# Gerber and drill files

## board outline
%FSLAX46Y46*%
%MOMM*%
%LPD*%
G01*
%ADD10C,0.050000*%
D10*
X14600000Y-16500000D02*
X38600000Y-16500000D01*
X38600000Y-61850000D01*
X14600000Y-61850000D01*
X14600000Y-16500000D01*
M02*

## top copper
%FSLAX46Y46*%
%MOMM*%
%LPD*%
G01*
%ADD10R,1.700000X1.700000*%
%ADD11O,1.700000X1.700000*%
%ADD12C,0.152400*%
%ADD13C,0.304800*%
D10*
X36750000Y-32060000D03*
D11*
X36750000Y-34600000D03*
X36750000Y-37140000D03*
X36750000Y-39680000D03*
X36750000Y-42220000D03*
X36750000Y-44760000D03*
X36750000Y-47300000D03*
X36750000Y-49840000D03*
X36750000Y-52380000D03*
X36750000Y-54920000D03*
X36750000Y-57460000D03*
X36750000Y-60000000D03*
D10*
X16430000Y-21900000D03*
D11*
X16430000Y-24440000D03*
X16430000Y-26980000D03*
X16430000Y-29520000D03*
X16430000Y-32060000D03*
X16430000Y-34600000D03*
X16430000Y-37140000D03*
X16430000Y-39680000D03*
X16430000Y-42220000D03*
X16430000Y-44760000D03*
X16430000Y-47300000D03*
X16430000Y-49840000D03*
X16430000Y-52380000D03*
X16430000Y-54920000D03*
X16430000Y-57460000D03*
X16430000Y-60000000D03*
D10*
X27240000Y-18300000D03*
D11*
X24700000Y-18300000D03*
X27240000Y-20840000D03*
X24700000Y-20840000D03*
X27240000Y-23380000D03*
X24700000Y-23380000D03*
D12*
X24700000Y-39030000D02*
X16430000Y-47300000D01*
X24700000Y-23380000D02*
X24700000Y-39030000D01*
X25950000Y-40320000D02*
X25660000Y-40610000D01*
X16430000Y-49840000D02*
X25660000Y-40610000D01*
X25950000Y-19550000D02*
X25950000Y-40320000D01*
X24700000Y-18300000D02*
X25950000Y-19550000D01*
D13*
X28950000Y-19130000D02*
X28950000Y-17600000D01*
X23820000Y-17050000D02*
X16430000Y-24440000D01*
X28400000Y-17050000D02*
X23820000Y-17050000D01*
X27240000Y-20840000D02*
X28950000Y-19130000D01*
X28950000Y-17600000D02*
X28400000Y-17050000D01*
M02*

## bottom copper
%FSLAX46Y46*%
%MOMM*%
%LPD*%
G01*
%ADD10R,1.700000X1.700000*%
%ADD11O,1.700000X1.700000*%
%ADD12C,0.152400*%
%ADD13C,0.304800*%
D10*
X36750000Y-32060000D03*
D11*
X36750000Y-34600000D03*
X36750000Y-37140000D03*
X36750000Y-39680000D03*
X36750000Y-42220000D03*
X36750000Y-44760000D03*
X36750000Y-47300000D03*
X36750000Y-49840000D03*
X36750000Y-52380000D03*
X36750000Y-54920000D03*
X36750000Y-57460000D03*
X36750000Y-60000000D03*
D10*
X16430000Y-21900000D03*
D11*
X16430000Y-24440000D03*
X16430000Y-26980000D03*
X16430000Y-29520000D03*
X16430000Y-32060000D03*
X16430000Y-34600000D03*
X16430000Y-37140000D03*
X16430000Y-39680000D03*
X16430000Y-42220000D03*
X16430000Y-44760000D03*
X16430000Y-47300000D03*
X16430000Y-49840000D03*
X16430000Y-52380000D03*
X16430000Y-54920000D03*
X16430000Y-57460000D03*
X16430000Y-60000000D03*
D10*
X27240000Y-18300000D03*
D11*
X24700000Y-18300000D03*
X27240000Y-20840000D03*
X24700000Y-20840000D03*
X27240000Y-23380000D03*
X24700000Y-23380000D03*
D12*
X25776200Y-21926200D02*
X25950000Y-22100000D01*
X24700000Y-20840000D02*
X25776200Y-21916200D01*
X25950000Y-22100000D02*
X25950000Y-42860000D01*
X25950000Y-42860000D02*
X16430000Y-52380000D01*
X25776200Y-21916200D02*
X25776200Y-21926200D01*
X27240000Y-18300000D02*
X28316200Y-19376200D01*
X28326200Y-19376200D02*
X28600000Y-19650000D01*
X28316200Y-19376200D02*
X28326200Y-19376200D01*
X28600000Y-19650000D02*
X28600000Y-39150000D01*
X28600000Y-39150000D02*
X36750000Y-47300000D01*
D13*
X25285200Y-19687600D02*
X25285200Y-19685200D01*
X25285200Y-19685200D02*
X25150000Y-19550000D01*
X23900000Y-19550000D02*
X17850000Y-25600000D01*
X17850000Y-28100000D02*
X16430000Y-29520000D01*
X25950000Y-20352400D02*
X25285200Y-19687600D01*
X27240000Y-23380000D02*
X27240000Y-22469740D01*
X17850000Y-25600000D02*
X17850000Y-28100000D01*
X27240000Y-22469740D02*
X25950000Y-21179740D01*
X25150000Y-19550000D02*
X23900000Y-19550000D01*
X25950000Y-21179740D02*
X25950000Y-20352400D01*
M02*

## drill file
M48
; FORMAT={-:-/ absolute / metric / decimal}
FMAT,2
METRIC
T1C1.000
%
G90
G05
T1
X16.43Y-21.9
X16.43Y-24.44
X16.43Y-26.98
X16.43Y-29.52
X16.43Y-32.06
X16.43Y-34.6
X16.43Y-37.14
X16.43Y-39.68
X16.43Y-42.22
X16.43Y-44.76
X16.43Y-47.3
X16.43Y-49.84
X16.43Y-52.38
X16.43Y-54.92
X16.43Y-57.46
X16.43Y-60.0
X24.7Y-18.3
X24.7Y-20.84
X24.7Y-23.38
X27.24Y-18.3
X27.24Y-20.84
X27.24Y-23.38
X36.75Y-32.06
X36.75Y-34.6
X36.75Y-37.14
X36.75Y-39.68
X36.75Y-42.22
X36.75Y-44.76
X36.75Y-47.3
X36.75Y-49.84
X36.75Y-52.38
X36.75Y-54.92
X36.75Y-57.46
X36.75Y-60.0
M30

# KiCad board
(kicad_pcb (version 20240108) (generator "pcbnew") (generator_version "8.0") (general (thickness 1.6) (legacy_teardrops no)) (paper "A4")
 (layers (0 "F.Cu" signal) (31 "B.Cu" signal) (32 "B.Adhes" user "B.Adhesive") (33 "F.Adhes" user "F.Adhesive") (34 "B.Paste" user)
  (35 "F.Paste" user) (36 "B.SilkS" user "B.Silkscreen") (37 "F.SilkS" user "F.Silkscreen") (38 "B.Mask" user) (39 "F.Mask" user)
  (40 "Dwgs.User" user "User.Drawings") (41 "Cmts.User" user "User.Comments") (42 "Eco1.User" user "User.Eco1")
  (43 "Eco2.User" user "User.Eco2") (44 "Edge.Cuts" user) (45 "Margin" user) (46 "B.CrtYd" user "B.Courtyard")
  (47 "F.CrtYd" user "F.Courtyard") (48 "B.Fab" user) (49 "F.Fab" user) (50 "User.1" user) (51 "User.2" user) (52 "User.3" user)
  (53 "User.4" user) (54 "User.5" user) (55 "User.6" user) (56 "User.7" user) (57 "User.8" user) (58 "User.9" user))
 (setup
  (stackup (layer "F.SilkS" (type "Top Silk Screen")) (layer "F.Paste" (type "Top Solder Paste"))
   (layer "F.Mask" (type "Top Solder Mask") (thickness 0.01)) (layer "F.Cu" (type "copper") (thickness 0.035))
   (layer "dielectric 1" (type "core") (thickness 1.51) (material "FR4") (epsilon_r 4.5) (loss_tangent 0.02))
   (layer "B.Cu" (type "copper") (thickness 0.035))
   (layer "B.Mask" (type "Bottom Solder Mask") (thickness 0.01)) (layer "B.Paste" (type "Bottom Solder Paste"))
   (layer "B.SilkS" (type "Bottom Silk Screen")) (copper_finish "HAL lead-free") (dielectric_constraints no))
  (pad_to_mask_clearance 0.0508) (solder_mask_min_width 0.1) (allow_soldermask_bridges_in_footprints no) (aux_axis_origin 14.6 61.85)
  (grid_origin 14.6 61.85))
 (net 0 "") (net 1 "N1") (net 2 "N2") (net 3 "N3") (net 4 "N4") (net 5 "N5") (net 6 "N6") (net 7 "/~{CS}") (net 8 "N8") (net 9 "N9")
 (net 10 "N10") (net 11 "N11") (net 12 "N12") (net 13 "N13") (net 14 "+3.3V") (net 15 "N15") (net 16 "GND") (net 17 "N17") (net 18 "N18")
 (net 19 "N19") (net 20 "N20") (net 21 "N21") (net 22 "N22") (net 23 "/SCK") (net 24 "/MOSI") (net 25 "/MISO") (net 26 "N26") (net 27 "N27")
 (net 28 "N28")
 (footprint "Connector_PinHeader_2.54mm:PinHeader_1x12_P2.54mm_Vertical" (layer "F.Cu") (at 36.75 32.06)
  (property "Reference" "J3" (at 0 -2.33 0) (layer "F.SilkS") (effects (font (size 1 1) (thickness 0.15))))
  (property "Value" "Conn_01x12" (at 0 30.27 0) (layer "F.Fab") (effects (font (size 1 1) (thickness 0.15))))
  (pad "1" thru_hole rect (at 0 0) (size 1.7 1.7) (drill 1) (layers "*.Cu" "*.Mask") (remove_unused_layers no) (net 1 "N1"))
  (pad "2" thru_hole oval (at 0 2.54) (size 1.7 1.7) (drill 1) (layers "*.Cu" "*.Mask") (remove_unused_layers no) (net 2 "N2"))
  (pad "3" thru_hole oval (at 0 5.08) (size 1.7 1.7) (drill 1) (layers "*.Cu" "*.Mask") (remove_unused_layers no) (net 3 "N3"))
  (pad "4" thru_hole oval (at 0 7.62) (size 1.7 1.7) (drill 1) (layers "*.Cu" "*.Mask") (remove_unused_layers no) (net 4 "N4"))
  (pad "5" thru_hole oval (at 0 10.16) (size 1.7 1.7) (drill 1) (layers "*.Cu" "*.Mask") (remove_unused_layers no) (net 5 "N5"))
  (pad "6" thru_hole oval (at 0 12.7) (size 1.7 1.7) (drill 1) (layers "*.Cu" "*.Mask") (remove_unused_layers no) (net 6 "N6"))
  (pad "7" thru_hole oval (at 0 15.24) (size 1.7 1.7) (drill 1) (layers "*.Cu" "*.Mask") (remove_unused_layers no) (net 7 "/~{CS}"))
  (pad "8" thru_hole oval (at 0 17.78) (size 1.7 1.7) (drill 1) (layers "*.Cu" "*.Mask") (remove_unused_layers no) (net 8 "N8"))
  (pad "9" thru_hole oval (at 0 20.32) (size 1.7 1.7) (drill 1) (layers "*.Cu" "*.Mask") (remove_unused_layers no) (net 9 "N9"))
  (pad "10" thru_hole oval (at 0 22.86) (size 1.7 1.7) (drill 1) (layers "*.Cu" "*.Mask") (remove_unused_layers no) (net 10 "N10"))
  (pad "11" thru_hole oval (at 0 25.4) (size 1.7 1.7) (drill 1) (layers "*.Cu" "*.Mask") (remove_unused_layers no) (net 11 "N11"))
  (pad "12" thru_hole oval (at 0 27.94) (size 1.7 1.7) (drill 1) (layers "*.Cu" "*.Mask") (remove_unused_layers no) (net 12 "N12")))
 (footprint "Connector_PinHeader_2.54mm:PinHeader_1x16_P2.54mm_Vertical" (layer "F.Cu") (at 16.43 21.9)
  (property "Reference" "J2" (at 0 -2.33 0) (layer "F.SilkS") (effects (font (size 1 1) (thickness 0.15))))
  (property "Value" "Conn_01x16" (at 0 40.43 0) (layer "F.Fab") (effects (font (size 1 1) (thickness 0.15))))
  (pad "1" thru_hole rect (at 0 0) (size 1.7 1.7) (drill 1) (layers "*.Cu" "*.Mask") (remove_unused_layers no) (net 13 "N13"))
  (pad "2" thru_hole oval (at 0 2.54) (size 1.7 1.7) (drill 1) (layers "*.Cu" "*.Mask") (remove_unused_layers no) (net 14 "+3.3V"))
  (pad "3" thru_hole oval (at 0 5.08) (size 1.7 1.7) (drill 1) (layers "*.Cu" "*.Mask") (remove_unused_layers no) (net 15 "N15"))
  (pad "4" thru_hole oval (at 0 7.62) (size 1.7 1.7) (drill 1) (layers "*.Cu" "*.Mask") (remove_unused_layers no) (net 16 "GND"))
  (pad "5" thru_hole oval (at 0 10.16) (size 1.7 1.7) (drill 1) (layers "*.Cu" "*.Mask") (remove_unused_layers no) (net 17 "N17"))
  (pad "6" thru_hole oval (at 0 12.7) (size 1.7 1.7) (drill 1) (layers "*.Cu" "*.Mask") (remove_unused_layers no) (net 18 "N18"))
  (pad "7" thru_hole oval (at 0 15.24) (size 1.7 1.7) (drill 1) (layers "*.Cu" "*.Mask") (remove_unused_layers no) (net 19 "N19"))
  (pad "8" thru_hole oval (at 0 17.78) (size 1.7 1.7) (drill 1) (layers "*.Cu" "*.Mask") (remove_unused_layers no) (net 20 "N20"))
  (pad "9" thru_hole oval (at 0 20.32) (size 1.7 1.7) (drill 1) (layers "*.Cu" "*.Mask") (remove_unused_layers no) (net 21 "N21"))
  (pad "10" thru_hole oval (at 0 22.86) (size 1.7 1.7) (drill 1) (layers "*.Cu" "*.Mask") (remove_unused_layers no) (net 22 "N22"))
  (pad "11" thru_hole oval (at 0 25.4) (size 1.7 1.7) (drill 1) (layers "*.Cu" "*.Mask") (remove_unused_layers no) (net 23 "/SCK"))
  (pad "12" thru_hole oval (at 0 27.94) (size 1.7 1.7) (drill 1) (layers "*.Cu" "*.Mask") (remove_unused_layers no) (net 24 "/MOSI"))
  (pad "13" thru_hole oval (at 0 30.48) (size 1.7 1.7) (drill 1) (layers "*.Cu" "*.Mask") (remove_unused_layers no) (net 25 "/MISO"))
  (pad "14" thru_hole oval (at 0 33.02) (size 1.7 1.7) (drill 1) (layers "*.Cu" "*.Mask") (remove_unused_layers no) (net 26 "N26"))
  (pad "15" thru_hole oval (at 0 35.56) (size 1.7 1.7) (drill 1) (layers "*.Cu" "*.Mask") (remove_unused_layers no) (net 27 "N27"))
  (pad "16" thru_hole oval (at 0 38.1) (size 1.7 1.7) (drill 1) (layers "*.Cu" "*.Mask") (remove_unused_layers no) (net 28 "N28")))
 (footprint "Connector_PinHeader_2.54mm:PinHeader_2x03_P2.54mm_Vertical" (layer "B.Cu") (at 27.24 18.3 180)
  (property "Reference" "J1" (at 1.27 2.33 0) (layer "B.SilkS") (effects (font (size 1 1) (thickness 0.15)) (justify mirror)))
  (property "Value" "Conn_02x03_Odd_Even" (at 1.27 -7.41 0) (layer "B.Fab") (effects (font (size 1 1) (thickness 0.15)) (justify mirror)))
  (pad "1" thru_hole rect (at 0 0 180) (size 1.7 1.7) (drill 1) (layers "*.Cu" "*.Mask") (remove_unused_layers no) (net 7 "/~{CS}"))
  (pad "2" thru_hole oval (at 2.54 0 180) (size 1.7 1.7) (drill 1) (layers "*.Cu" "*.Mask") (remove_unused_layers no) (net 24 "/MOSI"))
  (pad "3" thru_hole oval (at 0 -2.54 180) (size 1.7 1.7) (drill 1) (layers "*.Cu" "*.Mask") (remove_unused_layers no) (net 14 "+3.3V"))
  (pad "4" thru_hole oval (at 2.54 -2.54 180) (size 1.7 1.7) (drill 1) (layers "*.Cu" "*.Mask") (remove_unused_layers no) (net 25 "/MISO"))
  (pad "5" thru_hole oval (at 0 -5.08 180) (size 1.7 1.7) (drill 1) (layers "*.Cu" "*.Mask") (remove_unused_layers no) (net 16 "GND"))
  (pad "6" thru_hole oval (at 2.54 -5.08 180) (size 1.7 1.7) (drill 1) (layers "*.Cu" "*.Mask") (remove_unused_layers no) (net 23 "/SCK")))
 (gr_rect (start 14.6 16.5) (end 38.6 61.85) (stroke (width 0.05) (type default)) (fill none) (layer "Edge.Cuts"))
 (segment (start 25.7762 21.9262) (end 25.95 22.1) (width 0.1524) (layer "B.Cu") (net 25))
 (segment (start 24.7 20.84) (end 25.7762 21.9162) (width 0.1524) (layer "B.Cu") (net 25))
 (segment (start 25.95 22.1) (end 25.95 42.86) (width 0.1524) (layer "B.Cu") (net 25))
 (segment (start 25.95 42.86) (end 16.43 52.38) (width 0.1524) (layer "B.Cu") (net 25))
 (segment (start 25.7762 21.9162) (end 25.7762 21.9262) (width 0.1524) (layer "B.Cu") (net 25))
 (segment (start 24.7 39.03) (end 16.43 47.3) (width 0.1524) (layer "F.Cu") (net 23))
 (segment (start 24.7 23.38) (end 24.7 39.03) (width 0.1524) (layer "F.Cu") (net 23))
 (segment (start 25.95 40.32) (end 25.66 40.61) (width 0.1524) (layer "F.Cu") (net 24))
 (segment (start 16.43 49.84) (end 25.66 40.61) (width 0.1524) (layer "F.Cu") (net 24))
 (segment (start 25.95 19.55) (end 25.95 40.32) (width 0.1524) (layer "F.Cu") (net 24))
 (segment (start 24.7 18.3) (end 25.95 19.55) (width 0.1524) (layer "F.Cu") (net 24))
 (segment (start 27.24 18.3) (end 28.3162 19.3762) (width 0.1524) (layer "B.Cu") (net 7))
 (segment (start 28.3262 19.3762) (end 28.6 19.65) (width 0.1524) (layer "B.Cu") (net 7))
 (segment (start 28.3162 19.3762) (end 28.3262 19.3762) (width 0.1524) (layer "B.Cu") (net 7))
 (segment (start 28.6 19.65) (end 28.6 39.15) (width 0.1524) (layer "B.Cu") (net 7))
 (segment (start 28.6 39.15) (end 36.75 47.3) (width 0.1524) (layer "B.Cu") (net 7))
 (segment (start 25.2852 19.6876) (end 25.2852 19.6852) (width 0.3048) (layer "B.Cu") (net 16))
 (segment (start 25.2852 19.6852) (end 25.15 19.55) (width 0.3048) (layer "B.Cu") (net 16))
 (segment (start 23.9 19.55) (end 17.85 25.6) (width 0.3048) (layer "B.Cu") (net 16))
 (segment (start 17.85 28.1) (end 16.43 29.52) (width 0.3048) (layer "B.Cu") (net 16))
 (segment (start 25.95 20.3524) (end 25.2852 19.6876) (width 0.3048) (layer "B.Cu") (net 16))
 (segment (start 27.24 23.38) (end 27.24 22.46974) (width 0.3048) (layer "B.Cu") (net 16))
 (segment (start 17.85 25.6) (end 17.85 28.1) (width 0.3048) (layer "B.Cu") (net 16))
 (segment (start 27.24 22.46974) (end 25.95 21.17974) (width 0.3048) (layer "B.Cu") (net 16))
 (segment (start 25.15 19.55) (end 23.9 19.55) (width 0.3048) (layer "B.Cu") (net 16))
 (segment (start 25.95 21.17974) (end 25.95 20.3524) (width 0.3048) (layer "B.Cu") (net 16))
 (segment (start 28.95 19.13) (end 28.95 17.6) (width 0.3048) (layer "F.Cu") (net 14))
 (segment (start 23.82 17.05) (end 16.43 24.44) (width 0.3048) (layer "F.Cu") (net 14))
 (segment (start 28.4 17.05) (end 23.82 17.05) (width 0.3048) (layer "F.Cu") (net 14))
 (segment (start 27.24 20.84) (end 28.95 19.13) (width 0.3048) (layer "F.Cu") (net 14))
 (segment (start 28.95 17.6) (end 28.4 17.05) (width 0.3048) (layer "F.Cu") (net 14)))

